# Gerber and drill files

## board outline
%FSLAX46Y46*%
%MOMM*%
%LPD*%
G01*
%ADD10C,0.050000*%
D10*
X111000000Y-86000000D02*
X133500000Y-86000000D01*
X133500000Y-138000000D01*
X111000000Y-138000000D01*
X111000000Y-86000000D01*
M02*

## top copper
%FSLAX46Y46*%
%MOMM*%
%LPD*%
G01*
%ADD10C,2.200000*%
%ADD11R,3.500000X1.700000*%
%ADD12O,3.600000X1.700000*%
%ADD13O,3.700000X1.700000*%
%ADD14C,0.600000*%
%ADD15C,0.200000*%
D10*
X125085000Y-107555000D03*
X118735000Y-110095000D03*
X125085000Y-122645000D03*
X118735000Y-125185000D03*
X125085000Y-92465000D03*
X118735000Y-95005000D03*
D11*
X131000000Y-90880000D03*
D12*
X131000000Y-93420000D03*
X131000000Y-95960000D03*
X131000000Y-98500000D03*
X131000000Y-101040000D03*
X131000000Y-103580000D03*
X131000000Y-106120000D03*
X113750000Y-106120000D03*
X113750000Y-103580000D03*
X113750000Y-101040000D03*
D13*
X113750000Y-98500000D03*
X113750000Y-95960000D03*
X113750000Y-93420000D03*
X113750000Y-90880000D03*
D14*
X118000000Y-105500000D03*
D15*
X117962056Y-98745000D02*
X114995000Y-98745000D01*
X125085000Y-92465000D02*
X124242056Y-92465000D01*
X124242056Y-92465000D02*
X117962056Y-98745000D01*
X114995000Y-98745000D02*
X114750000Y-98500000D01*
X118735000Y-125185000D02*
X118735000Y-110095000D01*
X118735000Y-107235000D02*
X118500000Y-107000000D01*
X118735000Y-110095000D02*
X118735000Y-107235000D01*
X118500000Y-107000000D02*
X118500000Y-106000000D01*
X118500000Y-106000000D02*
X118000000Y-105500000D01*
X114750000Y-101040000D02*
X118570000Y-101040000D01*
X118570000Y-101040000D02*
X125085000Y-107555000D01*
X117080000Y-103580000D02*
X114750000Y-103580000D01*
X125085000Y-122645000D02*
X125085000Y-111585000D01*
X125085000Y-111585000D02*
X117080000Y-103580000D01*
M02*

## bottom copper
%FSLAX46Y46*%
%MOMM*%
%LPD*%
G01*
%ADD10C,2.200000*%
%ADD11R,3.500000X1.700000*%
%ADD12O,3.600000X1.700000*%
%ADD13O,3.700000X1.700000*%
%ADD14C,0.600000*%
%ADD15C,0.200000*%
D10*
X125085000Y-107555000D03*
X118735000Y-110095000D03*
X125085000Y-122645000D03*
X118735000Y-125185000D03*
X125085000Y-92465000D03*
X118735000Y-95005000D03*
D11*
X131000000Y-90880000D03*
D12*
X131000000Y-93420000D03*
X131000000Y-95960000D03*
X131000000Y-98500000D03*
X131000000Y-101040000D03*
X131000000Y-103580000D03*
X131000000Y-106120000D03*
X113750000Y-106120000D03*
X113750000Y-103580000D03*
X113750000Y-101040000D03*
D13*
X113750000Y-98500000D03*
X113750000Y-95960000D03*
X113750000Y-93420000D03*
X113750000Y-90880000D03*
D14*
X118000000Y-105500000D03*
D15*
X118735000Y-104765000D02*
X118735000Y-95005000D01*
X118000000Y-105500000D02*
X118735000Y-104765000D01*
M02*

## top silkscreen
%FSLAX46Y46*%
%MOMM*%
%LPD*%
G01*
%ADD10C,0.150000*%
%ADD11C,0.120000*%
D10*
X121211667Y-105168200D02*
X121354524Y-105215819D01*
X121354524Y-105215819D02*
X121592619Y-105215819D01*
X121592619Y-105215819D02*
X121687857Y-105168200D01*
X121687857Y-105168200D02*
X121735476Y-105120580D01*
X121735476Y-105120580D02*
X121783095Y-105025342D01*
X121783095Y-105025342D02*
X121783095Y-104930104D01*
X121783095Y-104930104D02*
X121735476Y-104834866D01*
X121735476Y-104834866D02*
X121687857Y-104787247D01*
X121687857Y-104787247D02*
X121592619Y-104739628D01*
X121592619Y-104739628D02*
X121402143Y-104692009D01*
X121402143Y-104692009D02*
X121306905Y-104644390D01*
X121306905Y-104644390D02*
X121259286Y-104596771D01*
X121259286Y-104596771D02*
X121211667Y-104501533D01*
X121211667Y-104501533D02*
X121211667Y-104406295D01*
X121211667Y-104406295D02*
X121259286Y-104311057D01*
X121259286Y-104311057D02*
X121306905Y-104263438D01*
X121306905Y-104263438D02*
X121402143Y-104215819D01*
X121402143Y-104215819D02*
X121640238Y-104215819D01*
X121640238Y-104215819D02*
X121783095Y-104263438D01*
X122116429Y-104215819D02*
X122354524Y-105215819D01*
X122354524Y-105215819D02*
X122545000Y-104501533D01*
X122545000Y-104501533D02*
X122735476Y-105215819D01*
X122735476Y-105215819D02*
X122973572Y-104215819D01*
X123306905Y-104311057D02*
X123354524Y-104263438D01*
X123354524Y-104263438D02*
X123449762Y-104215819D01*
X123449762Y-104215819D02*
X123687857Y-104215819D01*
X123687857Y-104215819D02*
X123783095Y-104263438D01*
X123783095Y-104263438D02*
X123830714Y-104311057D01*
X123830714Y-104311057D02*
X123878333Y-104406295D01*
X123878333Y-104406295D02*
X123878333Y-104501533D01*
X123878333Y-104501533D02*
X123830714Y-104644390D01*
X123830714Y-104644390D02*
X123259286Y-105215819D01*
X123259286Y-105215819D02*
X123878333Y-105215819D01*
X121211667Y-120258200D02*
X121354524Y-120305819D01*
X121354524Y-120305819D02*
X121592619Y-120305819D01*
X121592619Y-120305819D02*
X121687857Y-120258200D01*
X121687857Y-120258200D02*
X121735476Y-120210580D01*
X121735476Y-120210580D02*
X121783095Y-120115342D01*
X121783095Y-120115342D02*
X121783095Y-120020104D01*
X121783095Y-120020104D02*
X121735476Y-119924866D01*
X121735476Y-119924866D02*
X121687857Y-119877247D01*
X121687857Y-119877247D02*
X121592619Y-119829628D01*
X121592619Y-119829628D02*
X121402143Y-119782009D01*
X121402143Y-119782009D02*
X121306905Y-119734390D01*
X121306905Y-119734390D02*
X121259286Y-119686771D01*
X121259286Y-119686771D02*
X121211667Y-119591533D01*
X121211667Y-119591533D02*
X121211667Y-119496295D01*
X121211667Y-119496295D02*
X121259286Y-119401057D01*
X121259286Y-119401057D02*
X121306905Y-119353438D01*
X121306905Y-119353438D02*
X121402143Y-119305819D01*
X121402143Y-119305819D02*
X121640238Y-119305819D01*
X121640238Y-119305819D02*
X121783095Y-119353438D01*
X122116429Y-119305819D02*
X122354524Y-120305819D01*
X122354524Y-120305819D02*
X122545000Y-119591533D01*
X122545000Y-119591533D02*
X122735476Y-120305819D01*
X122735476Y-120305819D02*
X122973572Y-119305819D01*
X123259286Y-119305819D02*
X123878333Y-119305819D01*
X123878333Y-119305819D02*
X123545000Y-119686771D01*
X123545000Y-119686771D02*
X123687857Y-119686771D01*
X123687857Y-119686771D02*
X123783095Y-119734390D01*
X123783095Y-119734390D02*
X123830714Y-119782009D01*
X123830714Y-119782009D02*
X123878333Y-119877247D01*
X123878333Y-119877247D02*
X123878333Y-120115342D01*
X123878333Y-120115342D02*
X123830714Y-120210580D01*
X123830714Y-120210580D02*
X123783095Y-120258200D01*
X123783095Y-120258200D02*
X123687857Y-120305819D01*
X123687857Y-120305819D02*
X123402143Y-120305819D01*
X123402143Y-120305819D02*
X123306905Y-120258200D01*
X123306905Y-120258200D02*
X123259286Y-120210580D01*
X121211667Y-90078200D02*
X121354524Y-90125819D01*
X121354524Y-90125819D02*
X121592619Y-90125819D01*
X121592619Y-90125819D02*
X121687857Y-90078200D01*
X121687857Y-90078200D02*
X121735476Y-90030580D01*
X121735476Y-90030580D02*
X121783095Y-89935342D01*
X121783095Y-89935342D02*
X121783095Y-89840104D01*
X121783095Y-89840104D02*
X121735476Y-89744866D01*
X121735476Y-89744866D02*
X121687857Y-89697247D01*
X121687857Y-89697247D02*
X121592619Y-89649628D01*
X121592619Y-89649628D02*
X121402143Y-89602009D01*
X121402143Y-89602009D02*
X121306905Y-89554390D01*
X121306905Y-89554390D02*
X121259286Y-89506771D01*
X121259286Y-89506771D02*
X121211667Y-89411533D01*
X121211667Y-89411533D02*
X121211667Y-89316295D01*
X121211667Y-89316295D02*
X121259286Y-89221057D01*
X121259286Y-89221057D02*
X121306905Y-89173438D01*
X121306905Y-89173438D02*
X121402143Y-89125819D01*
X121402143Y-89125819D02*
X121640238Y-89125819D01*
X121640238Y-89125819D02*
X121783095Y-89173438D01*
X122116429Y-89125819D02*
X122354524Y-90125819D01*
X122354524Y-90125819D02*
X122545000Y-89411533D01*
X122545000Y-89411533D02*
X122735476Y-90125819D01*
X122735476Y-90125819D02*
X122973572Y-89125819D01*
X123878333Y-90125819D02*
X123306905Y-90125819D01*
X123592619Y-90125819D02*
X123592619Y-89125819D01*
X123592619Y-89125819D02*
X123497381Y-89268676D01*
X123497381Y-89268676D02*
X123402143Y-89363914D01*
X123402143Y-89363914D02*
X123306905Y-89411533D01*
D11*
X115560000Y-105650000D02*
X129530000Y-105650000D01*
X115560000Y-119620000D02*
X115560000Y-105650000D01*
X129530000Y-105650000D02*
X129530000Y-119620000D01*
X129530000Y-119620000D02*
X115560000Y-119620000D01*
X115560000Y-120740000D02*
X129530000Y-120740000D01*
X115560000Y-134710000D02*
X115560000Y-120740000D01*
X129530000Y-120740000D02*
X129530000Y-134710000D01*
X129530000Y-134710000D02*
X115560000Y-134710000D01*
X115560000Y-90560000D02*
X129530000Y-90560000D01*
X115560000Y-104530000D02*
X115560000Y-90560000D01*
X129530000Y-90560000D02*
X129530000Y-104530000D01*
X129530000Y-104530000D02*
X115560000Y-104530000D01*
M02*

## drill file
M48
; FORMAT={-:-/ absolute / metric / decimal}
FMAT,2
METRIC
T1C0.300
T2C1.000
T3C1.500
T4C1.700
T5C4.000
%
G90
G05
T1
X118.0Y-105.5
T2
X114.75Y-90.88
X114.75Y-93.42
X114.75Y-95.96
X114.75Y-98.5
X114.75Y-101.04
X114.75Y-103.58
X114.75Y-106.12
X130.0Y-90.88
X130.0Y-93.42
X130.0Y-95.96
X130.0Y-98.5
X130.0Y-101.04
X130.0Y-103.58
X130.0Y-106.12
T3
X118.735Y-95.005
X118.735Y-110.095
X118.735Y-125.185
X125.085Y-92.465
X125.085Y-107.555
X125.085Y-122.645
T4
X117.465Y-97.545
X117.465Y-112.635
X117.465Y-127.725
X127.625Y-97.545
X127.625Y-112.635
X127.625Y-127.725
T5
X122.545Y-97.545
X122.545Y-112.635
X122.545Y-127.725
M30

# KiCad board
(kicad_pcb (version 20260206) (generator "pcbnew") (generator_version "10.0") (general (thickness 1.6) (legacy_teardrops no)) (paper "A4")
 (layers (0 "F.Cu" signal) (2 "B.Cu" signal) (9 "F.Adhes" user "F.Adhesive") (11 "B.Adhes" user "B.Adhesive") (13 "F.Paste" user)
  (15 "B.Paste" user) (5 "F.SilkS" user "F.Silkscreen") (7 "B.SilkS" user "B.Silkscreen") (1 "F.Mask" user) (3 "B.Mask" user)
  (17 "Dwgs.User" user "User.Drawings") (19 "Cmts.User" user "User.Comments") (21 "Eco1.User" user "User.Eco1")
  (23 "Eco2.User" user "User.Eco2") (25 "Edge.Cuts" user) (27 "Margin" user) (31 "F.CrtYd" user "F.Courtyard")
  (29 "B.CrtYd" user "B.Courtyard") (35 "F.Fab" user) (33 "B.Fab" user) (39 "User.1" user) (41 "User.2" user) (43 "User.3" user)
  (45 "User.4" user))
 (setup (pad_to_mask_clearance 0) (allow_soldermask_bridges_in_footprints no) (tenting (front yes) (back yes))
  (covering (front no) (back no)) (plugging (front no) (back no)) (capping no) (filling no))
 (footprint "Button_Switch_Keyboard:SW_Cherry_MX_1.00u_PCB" (layer "F.Cu") (at 125.085 107.555)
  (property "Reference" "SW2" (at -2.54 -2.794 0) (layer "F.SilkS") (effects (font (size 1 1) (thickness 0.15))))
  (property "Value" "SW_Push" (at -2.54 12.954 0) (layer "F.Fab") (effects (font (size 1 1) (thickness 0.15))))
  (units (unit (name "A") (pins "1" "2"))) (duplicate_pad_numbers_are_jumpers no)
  (fp_line (start -9.525 -1.905) (end 4.445 -1.905) (stroke (width 0.12) (type solid)) (layer "F.SilkS"))
  (fp_line (start -9.525 12.065) (end -9.525 -1.905) (stroke (width 0.12) (type solid)) (layer "F.SilkS"))
  (fp_line (start 4.445 -1.905) (end 4.445 12.065) (stroke (width 0.12) (type solid)) (layer "F.SilkS"))
  (fp_line (start 4.445 12.065) (end -9.525 12.065) (stroke (width 0.12) (type solid)) (layer "F.SilkS"))
  (pad "" np_thru_hole circle (at -7.62 5.08) (size 1.7 1.7) (drill 1.7) (layers "*.Cu" "*.Mask"))
  (pad "" np_thru_hole circle (at -2.54 5.08) (size 4 4) (drill 4) (layers "*.Cu" "*.Mask"))
  (pad "" np_thru_hole circle (at 2.54 5.08) (size 1.7 1.7) (drill 1.7) (layers "*.Cu" "*.Mask"))
  (pad "1" thru_hole circle (at 0 0) (size 2.2 2.2) (drill 1.5) (layers "*.Cu" "*.Mask") (remove_unused_layers no)
   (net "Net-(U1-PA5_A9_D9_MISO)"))
  (pad "2" thru_hole circle (at -6.35 2.54) (size 2.2 2.2) (drill 1.5) (layers "*.Cu" "*.Mask") (remove_unused_layers no) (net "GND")))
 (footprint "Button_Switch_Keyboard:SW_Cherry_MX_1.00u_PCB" (layer "F.Cu") (at 125.085 122.645)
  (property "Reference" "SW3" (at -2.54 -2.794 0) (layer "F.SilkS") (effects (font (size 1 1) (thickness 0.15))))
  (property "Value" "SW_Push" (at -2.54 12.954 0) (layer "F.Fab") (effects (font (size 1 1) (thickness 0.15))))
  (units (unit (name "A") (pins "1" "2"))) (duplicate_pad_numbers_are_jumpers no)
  (fp_line (start -9.525 -1.905) (end 4.445 -1.905) (stroke (width 0.12) (type solid)) (layer "F.SilkS"))
  (fp_line (start -9.525 12.065) (end -9.525 -1.905) (stroke (width 0.12) (type solid)) (layer "F.SilkS"))
  (fp_line (start 4.445 -1.905) (end 4.445 12.065) (stroke (width 0.12) (type solid)) (layer "F.SilkS"))
  (fp_line (start 4.445 12.065) (end -9.525 12.065) (stroke (width 0.12) (type solid)) (layer "F.SilkS"))
  (pad "" np_thru_hole circle (at -7.62 5.08) (size 1.7 1.7) (drill 1.7) (layers "*.Cu" "*.Mask"))
  (pad "" np_thru_hole circle (at -2.54 5.08) (size 4 4) (drill 4) (layers "*.Cu" "*.Mask"))
  (pad "" np_thru_hole circle (at 2.54 5.08) (size 1.7 1.7) (drill 1.7) (layers "*.Cu" "*.Mask"))
  (pad "1" thru_hole circle (at 0 0) (size 2.2 2.2) (drill 1.5) (layers "*.Cu" "*.Mask") (remove_unused_layers no)
   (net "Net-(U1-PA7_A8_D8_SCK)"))
  (pad "2" thru_hole circle (at -6.35 2.54) (size 2.2 2.2) (drill 1.5) (layers "*.Cu" "*.Mask") (remove_unused_layers no) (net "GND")))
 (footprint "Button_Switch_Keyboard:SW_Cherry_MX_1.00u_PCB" (layer "F.Cu") (at 125.085 92.465)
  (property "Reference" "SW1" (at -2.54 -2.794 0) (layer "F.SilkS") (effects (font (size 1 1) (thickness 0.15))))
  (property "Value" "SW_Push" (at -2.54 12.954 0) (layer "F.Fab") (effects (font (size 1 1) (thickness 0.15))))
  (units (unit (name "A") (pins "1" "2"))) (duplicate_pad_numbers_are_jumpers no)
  (fp_line (start -9.525 -1.905) (end 4.445 -1.905) (stroke (width 0.12) (type solid)) (layer "F.SilkS"))
  (fp_line (start -9.525 12.065) (end -9.525 -1.905) (stroke (width 0.12) (type solid)) (layer "F.SilkS"))
  (fp_line (start 4.445 -1.905) (end 4.445 12.065) (stroke (width 0.12) (type solid)) (layer "F.SilkS"))
  (fp_line (start 4.445 12.065) (end -9.525 12.065) (stroke (width 0.12) (type solid)) (layer "F.SilkS"))
  (pad "" np_thru_hole circle (at -7.62 5.08) (size 1.7 1.7) (drill 1.7) (layers "*.Cu" "*.Mask"))
  (pad "" np_thru_hole circle (at -2.54 5.08) (size 4 4) (drill 4) (layers "*.Cu" "*.Mask"))
  (pad "" np_thru_hole circle (at 2.54 5.08) (size 1.7 1.7) (drill 1.7) (layers "*.Cu" "*.Mask"))
  (pad "1" thru_hole circle (at 0 0) (size 2.2 2.2) (drill 1.5) (layers "*.Cu" "*.Mask") (remove_unused_layers no)
   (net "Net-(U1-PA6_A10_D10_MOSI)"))
  (pad "2" thru_hole circle (at -6.35 2.54) (size 2.2 2.2) (drill 1.5) (layers "*.Cu" "*.Mask") (remove_unused_layers no) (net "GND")))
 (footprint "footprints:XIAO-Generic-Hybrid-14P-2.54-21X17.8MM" (layer "B.Cu") (at 122.375 98.5 180)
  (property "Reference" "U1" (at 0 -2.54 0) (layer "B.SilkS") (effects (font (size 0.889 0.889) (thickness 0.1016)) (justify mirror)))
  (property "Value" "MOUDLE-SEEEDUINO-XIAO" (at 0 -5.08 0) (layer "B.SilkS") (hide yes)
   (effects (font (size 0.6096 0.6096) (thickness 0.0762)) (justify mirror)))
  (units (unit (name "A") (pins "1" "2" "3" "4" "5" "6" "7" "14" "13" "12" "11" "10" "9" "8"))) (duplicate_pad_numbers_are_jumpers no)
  (pad "1" thru_hole rect (at -7.625 7.62 180) (size 3.5 1.7) (drill 1 (offset -1 0)) (layers "*.Cu" "*.Mask") (remove_unused_layers no)
   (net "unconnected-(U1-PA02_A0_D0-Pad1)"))
  (pad "2" thru_hole oval (at -7.625 5.08 180) (size 3.6 1.7) (drill 1 (offset -1 0)) (layers "*.Cu" "*.Mask") (remove_unused_layers no)
   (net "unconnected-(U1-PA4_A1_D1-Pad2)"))
  (pad "3" thru_hole oval (at -7.625 2.54 180) (size 3.6 1.7) (drill 1 (offset -1 0)) (layers "*.Cu" "*.Mask") (remove_unused_layers no)
   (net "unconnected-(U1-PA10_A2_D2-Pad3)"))
  (pad "4" thru_hole oval (at -7.625 0 180) (size 3.6 1.7) (drill 1 (offset -1 0)) (layers "*.Cu" "*.Mask") (remove_unused_layers no)
   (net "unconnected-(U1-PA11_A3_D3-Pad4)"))
  (pad "5" thru_hole oval (at -7.625 -2.54 180) (size 3.6 1.7) (drill 1 (offset -1 0)) (layers "*.Cu" "*.Mask") (remove_unused_layers no)
   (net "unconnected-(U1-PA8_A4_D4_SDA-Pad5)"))
  (pad "6" thru_hole oval (at -7.625 -5.08) (size 3.6 1.7) (drill 1 (offset 1 0)) (layers "*.Cu" "*.Mask") (remove_unused_layers no)
   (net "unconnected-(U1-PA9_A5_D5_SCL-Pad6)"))
  (pad "7" thru_hole oval (at -7.625 -7.62 180) (size 3.6 1.7) (drill 1 (offset -1 0)) (layers "*.Cu" "*.Mask") (remove_unused_layers no)
   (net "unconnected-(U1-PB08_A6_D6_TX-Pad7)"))
  (pad "8" thru_hole oval (at 7.625 -7.62 180) (size 3.6 1.7) (drill 1 (offset 1 0)) (layers "*.Cu" "*.Mask") (remove_unused_layers no)
   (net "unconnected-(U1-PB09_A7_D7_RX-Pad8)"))
  (pad "9" thru_hole oval (at 7.625 -5.08 180) (size 3.6 1.7) (drill 1 (offset 1 0)) (layers "*.Cu" "*.Mask") (remove_unused_layers no)
   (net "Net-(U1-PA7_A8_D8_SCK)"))
  (pad "10" thru_hole oval (at 7.625 -2.54 180) (size 3.6 1.7) (drill 1 (offset 1 0)) (layers "*.Cu" "*.Mask") (remove_unused_layers no)
   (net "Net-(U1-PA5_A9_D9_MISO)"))
  (pad "11" thru_hole oval (at 7.625 0 180) (size 3.7 1.7) (drill 1 (offset 1 0)) (layers "*.Cu" "*.Mask") (remove_unused_layers no)
   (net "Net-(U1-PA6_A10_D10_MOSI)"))
  (pad "12" thru_hole oval (at 7.625 2.54 180) (size 3.7 1.7) (drill 1 (offset 1 0)) (layers "*.Cu" "*.Mask") (remove_unused_layers no)
   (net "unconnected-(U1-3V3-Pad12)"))
  (pad "13" thru_hole oval (at 7.625 5.08 180) (size 3.7 1.7) (drill 1 (offset 1 0)) (layers "*.Cu" "*.Mask") (remove_unused_layers no)
   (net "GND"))
  (pad "14" thru_hole oval (at 7.625 7.62 180) (size 3.7 1.7) (drill 1 (offset 1 0)) (layers "*.Cu" "*.Mask") (remove_unused_layers no)
   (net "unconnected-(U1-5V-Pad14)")))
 (gr_rect (start 111 86) (end 133.5 138) (stroke (width 0.05) (type default)) (fill no) (layer "Edge.Cuts"))
 (segment (start 117.962056 98.745) (end 114.995 98.745) (width 0.2) (layer "F.Cu") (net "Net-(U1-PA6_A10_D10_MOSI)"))
 (segment (start 125.085 92.465) (end 124.242056 92.465) (width 0.2) (layer "F.Cu") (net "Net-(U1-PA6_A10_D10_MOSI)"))
 (segment (start 124.242056 92.465) (end 117.962056 98.745) (width 0.2) (layer "F.Cu") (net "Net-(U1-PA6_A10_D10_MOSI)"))
 (segment (start 114.995 98.745) (end 114.75 98.5) (width 0.2) (layer "F.Cu") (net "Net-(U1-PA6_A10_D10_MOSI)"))
 (segment (start 118.735 125.185) (end 118.735 110.095) (width 0.2) (layer "F.Cu") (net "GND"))
 (segment (start 118.735 107.235) (end 118.5 107) (width 0.2) (layer "F.Cu") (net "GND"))
 (segment (start 118.735 110.095) (end 118.735 107.235) (width 0.2) (layer "F.Cu") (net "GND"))
 (segment (start 118.5 107) (end 118.5 106) (width 0.2) (layer "F.Cu") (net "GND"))
 (segment (start 118.5 106) (end 118 105.5) (width 0.2) (layer "F.Cu") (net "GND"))
 (via (at 118 105.5) (size 0.6) (drill 0.3) (layers "F.Cu" "B.Cu") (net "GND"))
 (segment (start 118.735 104.765) (end 118.735 95.005) (width 0.2) (layer "B.Cu") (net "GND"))
 (segment (start 118 105.5) (end 118.735 104.765) (width 0.2) (layer "B.Cu") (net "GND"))
 (segment (start 114.75 101.04) (end 118.57 101.04) (width 0.2) (layer "F.Cu") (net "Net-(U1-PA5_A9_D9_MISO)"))
 (segment (start 118.57 101.04) (end 125.085 107.555) (width 0.2) (layer "F.Cu") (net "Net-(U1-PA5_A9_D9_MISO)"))
 (segment (start 117.08 103.58) (end 114.75 103.58) (width 0.2) (layer "F.Cu") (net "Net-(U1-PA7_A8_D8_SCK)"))
 (segment (start 125.085 122.645) (end 125.085 111.585) (width 0.2) (layer "F.Cu") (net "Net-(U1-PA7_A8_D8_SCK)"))
 (segment (start 125.085 111.585) (end 117.08 103.58) (width 0.2) (layer "F.Cu") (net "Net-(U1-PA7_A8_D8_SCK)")))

